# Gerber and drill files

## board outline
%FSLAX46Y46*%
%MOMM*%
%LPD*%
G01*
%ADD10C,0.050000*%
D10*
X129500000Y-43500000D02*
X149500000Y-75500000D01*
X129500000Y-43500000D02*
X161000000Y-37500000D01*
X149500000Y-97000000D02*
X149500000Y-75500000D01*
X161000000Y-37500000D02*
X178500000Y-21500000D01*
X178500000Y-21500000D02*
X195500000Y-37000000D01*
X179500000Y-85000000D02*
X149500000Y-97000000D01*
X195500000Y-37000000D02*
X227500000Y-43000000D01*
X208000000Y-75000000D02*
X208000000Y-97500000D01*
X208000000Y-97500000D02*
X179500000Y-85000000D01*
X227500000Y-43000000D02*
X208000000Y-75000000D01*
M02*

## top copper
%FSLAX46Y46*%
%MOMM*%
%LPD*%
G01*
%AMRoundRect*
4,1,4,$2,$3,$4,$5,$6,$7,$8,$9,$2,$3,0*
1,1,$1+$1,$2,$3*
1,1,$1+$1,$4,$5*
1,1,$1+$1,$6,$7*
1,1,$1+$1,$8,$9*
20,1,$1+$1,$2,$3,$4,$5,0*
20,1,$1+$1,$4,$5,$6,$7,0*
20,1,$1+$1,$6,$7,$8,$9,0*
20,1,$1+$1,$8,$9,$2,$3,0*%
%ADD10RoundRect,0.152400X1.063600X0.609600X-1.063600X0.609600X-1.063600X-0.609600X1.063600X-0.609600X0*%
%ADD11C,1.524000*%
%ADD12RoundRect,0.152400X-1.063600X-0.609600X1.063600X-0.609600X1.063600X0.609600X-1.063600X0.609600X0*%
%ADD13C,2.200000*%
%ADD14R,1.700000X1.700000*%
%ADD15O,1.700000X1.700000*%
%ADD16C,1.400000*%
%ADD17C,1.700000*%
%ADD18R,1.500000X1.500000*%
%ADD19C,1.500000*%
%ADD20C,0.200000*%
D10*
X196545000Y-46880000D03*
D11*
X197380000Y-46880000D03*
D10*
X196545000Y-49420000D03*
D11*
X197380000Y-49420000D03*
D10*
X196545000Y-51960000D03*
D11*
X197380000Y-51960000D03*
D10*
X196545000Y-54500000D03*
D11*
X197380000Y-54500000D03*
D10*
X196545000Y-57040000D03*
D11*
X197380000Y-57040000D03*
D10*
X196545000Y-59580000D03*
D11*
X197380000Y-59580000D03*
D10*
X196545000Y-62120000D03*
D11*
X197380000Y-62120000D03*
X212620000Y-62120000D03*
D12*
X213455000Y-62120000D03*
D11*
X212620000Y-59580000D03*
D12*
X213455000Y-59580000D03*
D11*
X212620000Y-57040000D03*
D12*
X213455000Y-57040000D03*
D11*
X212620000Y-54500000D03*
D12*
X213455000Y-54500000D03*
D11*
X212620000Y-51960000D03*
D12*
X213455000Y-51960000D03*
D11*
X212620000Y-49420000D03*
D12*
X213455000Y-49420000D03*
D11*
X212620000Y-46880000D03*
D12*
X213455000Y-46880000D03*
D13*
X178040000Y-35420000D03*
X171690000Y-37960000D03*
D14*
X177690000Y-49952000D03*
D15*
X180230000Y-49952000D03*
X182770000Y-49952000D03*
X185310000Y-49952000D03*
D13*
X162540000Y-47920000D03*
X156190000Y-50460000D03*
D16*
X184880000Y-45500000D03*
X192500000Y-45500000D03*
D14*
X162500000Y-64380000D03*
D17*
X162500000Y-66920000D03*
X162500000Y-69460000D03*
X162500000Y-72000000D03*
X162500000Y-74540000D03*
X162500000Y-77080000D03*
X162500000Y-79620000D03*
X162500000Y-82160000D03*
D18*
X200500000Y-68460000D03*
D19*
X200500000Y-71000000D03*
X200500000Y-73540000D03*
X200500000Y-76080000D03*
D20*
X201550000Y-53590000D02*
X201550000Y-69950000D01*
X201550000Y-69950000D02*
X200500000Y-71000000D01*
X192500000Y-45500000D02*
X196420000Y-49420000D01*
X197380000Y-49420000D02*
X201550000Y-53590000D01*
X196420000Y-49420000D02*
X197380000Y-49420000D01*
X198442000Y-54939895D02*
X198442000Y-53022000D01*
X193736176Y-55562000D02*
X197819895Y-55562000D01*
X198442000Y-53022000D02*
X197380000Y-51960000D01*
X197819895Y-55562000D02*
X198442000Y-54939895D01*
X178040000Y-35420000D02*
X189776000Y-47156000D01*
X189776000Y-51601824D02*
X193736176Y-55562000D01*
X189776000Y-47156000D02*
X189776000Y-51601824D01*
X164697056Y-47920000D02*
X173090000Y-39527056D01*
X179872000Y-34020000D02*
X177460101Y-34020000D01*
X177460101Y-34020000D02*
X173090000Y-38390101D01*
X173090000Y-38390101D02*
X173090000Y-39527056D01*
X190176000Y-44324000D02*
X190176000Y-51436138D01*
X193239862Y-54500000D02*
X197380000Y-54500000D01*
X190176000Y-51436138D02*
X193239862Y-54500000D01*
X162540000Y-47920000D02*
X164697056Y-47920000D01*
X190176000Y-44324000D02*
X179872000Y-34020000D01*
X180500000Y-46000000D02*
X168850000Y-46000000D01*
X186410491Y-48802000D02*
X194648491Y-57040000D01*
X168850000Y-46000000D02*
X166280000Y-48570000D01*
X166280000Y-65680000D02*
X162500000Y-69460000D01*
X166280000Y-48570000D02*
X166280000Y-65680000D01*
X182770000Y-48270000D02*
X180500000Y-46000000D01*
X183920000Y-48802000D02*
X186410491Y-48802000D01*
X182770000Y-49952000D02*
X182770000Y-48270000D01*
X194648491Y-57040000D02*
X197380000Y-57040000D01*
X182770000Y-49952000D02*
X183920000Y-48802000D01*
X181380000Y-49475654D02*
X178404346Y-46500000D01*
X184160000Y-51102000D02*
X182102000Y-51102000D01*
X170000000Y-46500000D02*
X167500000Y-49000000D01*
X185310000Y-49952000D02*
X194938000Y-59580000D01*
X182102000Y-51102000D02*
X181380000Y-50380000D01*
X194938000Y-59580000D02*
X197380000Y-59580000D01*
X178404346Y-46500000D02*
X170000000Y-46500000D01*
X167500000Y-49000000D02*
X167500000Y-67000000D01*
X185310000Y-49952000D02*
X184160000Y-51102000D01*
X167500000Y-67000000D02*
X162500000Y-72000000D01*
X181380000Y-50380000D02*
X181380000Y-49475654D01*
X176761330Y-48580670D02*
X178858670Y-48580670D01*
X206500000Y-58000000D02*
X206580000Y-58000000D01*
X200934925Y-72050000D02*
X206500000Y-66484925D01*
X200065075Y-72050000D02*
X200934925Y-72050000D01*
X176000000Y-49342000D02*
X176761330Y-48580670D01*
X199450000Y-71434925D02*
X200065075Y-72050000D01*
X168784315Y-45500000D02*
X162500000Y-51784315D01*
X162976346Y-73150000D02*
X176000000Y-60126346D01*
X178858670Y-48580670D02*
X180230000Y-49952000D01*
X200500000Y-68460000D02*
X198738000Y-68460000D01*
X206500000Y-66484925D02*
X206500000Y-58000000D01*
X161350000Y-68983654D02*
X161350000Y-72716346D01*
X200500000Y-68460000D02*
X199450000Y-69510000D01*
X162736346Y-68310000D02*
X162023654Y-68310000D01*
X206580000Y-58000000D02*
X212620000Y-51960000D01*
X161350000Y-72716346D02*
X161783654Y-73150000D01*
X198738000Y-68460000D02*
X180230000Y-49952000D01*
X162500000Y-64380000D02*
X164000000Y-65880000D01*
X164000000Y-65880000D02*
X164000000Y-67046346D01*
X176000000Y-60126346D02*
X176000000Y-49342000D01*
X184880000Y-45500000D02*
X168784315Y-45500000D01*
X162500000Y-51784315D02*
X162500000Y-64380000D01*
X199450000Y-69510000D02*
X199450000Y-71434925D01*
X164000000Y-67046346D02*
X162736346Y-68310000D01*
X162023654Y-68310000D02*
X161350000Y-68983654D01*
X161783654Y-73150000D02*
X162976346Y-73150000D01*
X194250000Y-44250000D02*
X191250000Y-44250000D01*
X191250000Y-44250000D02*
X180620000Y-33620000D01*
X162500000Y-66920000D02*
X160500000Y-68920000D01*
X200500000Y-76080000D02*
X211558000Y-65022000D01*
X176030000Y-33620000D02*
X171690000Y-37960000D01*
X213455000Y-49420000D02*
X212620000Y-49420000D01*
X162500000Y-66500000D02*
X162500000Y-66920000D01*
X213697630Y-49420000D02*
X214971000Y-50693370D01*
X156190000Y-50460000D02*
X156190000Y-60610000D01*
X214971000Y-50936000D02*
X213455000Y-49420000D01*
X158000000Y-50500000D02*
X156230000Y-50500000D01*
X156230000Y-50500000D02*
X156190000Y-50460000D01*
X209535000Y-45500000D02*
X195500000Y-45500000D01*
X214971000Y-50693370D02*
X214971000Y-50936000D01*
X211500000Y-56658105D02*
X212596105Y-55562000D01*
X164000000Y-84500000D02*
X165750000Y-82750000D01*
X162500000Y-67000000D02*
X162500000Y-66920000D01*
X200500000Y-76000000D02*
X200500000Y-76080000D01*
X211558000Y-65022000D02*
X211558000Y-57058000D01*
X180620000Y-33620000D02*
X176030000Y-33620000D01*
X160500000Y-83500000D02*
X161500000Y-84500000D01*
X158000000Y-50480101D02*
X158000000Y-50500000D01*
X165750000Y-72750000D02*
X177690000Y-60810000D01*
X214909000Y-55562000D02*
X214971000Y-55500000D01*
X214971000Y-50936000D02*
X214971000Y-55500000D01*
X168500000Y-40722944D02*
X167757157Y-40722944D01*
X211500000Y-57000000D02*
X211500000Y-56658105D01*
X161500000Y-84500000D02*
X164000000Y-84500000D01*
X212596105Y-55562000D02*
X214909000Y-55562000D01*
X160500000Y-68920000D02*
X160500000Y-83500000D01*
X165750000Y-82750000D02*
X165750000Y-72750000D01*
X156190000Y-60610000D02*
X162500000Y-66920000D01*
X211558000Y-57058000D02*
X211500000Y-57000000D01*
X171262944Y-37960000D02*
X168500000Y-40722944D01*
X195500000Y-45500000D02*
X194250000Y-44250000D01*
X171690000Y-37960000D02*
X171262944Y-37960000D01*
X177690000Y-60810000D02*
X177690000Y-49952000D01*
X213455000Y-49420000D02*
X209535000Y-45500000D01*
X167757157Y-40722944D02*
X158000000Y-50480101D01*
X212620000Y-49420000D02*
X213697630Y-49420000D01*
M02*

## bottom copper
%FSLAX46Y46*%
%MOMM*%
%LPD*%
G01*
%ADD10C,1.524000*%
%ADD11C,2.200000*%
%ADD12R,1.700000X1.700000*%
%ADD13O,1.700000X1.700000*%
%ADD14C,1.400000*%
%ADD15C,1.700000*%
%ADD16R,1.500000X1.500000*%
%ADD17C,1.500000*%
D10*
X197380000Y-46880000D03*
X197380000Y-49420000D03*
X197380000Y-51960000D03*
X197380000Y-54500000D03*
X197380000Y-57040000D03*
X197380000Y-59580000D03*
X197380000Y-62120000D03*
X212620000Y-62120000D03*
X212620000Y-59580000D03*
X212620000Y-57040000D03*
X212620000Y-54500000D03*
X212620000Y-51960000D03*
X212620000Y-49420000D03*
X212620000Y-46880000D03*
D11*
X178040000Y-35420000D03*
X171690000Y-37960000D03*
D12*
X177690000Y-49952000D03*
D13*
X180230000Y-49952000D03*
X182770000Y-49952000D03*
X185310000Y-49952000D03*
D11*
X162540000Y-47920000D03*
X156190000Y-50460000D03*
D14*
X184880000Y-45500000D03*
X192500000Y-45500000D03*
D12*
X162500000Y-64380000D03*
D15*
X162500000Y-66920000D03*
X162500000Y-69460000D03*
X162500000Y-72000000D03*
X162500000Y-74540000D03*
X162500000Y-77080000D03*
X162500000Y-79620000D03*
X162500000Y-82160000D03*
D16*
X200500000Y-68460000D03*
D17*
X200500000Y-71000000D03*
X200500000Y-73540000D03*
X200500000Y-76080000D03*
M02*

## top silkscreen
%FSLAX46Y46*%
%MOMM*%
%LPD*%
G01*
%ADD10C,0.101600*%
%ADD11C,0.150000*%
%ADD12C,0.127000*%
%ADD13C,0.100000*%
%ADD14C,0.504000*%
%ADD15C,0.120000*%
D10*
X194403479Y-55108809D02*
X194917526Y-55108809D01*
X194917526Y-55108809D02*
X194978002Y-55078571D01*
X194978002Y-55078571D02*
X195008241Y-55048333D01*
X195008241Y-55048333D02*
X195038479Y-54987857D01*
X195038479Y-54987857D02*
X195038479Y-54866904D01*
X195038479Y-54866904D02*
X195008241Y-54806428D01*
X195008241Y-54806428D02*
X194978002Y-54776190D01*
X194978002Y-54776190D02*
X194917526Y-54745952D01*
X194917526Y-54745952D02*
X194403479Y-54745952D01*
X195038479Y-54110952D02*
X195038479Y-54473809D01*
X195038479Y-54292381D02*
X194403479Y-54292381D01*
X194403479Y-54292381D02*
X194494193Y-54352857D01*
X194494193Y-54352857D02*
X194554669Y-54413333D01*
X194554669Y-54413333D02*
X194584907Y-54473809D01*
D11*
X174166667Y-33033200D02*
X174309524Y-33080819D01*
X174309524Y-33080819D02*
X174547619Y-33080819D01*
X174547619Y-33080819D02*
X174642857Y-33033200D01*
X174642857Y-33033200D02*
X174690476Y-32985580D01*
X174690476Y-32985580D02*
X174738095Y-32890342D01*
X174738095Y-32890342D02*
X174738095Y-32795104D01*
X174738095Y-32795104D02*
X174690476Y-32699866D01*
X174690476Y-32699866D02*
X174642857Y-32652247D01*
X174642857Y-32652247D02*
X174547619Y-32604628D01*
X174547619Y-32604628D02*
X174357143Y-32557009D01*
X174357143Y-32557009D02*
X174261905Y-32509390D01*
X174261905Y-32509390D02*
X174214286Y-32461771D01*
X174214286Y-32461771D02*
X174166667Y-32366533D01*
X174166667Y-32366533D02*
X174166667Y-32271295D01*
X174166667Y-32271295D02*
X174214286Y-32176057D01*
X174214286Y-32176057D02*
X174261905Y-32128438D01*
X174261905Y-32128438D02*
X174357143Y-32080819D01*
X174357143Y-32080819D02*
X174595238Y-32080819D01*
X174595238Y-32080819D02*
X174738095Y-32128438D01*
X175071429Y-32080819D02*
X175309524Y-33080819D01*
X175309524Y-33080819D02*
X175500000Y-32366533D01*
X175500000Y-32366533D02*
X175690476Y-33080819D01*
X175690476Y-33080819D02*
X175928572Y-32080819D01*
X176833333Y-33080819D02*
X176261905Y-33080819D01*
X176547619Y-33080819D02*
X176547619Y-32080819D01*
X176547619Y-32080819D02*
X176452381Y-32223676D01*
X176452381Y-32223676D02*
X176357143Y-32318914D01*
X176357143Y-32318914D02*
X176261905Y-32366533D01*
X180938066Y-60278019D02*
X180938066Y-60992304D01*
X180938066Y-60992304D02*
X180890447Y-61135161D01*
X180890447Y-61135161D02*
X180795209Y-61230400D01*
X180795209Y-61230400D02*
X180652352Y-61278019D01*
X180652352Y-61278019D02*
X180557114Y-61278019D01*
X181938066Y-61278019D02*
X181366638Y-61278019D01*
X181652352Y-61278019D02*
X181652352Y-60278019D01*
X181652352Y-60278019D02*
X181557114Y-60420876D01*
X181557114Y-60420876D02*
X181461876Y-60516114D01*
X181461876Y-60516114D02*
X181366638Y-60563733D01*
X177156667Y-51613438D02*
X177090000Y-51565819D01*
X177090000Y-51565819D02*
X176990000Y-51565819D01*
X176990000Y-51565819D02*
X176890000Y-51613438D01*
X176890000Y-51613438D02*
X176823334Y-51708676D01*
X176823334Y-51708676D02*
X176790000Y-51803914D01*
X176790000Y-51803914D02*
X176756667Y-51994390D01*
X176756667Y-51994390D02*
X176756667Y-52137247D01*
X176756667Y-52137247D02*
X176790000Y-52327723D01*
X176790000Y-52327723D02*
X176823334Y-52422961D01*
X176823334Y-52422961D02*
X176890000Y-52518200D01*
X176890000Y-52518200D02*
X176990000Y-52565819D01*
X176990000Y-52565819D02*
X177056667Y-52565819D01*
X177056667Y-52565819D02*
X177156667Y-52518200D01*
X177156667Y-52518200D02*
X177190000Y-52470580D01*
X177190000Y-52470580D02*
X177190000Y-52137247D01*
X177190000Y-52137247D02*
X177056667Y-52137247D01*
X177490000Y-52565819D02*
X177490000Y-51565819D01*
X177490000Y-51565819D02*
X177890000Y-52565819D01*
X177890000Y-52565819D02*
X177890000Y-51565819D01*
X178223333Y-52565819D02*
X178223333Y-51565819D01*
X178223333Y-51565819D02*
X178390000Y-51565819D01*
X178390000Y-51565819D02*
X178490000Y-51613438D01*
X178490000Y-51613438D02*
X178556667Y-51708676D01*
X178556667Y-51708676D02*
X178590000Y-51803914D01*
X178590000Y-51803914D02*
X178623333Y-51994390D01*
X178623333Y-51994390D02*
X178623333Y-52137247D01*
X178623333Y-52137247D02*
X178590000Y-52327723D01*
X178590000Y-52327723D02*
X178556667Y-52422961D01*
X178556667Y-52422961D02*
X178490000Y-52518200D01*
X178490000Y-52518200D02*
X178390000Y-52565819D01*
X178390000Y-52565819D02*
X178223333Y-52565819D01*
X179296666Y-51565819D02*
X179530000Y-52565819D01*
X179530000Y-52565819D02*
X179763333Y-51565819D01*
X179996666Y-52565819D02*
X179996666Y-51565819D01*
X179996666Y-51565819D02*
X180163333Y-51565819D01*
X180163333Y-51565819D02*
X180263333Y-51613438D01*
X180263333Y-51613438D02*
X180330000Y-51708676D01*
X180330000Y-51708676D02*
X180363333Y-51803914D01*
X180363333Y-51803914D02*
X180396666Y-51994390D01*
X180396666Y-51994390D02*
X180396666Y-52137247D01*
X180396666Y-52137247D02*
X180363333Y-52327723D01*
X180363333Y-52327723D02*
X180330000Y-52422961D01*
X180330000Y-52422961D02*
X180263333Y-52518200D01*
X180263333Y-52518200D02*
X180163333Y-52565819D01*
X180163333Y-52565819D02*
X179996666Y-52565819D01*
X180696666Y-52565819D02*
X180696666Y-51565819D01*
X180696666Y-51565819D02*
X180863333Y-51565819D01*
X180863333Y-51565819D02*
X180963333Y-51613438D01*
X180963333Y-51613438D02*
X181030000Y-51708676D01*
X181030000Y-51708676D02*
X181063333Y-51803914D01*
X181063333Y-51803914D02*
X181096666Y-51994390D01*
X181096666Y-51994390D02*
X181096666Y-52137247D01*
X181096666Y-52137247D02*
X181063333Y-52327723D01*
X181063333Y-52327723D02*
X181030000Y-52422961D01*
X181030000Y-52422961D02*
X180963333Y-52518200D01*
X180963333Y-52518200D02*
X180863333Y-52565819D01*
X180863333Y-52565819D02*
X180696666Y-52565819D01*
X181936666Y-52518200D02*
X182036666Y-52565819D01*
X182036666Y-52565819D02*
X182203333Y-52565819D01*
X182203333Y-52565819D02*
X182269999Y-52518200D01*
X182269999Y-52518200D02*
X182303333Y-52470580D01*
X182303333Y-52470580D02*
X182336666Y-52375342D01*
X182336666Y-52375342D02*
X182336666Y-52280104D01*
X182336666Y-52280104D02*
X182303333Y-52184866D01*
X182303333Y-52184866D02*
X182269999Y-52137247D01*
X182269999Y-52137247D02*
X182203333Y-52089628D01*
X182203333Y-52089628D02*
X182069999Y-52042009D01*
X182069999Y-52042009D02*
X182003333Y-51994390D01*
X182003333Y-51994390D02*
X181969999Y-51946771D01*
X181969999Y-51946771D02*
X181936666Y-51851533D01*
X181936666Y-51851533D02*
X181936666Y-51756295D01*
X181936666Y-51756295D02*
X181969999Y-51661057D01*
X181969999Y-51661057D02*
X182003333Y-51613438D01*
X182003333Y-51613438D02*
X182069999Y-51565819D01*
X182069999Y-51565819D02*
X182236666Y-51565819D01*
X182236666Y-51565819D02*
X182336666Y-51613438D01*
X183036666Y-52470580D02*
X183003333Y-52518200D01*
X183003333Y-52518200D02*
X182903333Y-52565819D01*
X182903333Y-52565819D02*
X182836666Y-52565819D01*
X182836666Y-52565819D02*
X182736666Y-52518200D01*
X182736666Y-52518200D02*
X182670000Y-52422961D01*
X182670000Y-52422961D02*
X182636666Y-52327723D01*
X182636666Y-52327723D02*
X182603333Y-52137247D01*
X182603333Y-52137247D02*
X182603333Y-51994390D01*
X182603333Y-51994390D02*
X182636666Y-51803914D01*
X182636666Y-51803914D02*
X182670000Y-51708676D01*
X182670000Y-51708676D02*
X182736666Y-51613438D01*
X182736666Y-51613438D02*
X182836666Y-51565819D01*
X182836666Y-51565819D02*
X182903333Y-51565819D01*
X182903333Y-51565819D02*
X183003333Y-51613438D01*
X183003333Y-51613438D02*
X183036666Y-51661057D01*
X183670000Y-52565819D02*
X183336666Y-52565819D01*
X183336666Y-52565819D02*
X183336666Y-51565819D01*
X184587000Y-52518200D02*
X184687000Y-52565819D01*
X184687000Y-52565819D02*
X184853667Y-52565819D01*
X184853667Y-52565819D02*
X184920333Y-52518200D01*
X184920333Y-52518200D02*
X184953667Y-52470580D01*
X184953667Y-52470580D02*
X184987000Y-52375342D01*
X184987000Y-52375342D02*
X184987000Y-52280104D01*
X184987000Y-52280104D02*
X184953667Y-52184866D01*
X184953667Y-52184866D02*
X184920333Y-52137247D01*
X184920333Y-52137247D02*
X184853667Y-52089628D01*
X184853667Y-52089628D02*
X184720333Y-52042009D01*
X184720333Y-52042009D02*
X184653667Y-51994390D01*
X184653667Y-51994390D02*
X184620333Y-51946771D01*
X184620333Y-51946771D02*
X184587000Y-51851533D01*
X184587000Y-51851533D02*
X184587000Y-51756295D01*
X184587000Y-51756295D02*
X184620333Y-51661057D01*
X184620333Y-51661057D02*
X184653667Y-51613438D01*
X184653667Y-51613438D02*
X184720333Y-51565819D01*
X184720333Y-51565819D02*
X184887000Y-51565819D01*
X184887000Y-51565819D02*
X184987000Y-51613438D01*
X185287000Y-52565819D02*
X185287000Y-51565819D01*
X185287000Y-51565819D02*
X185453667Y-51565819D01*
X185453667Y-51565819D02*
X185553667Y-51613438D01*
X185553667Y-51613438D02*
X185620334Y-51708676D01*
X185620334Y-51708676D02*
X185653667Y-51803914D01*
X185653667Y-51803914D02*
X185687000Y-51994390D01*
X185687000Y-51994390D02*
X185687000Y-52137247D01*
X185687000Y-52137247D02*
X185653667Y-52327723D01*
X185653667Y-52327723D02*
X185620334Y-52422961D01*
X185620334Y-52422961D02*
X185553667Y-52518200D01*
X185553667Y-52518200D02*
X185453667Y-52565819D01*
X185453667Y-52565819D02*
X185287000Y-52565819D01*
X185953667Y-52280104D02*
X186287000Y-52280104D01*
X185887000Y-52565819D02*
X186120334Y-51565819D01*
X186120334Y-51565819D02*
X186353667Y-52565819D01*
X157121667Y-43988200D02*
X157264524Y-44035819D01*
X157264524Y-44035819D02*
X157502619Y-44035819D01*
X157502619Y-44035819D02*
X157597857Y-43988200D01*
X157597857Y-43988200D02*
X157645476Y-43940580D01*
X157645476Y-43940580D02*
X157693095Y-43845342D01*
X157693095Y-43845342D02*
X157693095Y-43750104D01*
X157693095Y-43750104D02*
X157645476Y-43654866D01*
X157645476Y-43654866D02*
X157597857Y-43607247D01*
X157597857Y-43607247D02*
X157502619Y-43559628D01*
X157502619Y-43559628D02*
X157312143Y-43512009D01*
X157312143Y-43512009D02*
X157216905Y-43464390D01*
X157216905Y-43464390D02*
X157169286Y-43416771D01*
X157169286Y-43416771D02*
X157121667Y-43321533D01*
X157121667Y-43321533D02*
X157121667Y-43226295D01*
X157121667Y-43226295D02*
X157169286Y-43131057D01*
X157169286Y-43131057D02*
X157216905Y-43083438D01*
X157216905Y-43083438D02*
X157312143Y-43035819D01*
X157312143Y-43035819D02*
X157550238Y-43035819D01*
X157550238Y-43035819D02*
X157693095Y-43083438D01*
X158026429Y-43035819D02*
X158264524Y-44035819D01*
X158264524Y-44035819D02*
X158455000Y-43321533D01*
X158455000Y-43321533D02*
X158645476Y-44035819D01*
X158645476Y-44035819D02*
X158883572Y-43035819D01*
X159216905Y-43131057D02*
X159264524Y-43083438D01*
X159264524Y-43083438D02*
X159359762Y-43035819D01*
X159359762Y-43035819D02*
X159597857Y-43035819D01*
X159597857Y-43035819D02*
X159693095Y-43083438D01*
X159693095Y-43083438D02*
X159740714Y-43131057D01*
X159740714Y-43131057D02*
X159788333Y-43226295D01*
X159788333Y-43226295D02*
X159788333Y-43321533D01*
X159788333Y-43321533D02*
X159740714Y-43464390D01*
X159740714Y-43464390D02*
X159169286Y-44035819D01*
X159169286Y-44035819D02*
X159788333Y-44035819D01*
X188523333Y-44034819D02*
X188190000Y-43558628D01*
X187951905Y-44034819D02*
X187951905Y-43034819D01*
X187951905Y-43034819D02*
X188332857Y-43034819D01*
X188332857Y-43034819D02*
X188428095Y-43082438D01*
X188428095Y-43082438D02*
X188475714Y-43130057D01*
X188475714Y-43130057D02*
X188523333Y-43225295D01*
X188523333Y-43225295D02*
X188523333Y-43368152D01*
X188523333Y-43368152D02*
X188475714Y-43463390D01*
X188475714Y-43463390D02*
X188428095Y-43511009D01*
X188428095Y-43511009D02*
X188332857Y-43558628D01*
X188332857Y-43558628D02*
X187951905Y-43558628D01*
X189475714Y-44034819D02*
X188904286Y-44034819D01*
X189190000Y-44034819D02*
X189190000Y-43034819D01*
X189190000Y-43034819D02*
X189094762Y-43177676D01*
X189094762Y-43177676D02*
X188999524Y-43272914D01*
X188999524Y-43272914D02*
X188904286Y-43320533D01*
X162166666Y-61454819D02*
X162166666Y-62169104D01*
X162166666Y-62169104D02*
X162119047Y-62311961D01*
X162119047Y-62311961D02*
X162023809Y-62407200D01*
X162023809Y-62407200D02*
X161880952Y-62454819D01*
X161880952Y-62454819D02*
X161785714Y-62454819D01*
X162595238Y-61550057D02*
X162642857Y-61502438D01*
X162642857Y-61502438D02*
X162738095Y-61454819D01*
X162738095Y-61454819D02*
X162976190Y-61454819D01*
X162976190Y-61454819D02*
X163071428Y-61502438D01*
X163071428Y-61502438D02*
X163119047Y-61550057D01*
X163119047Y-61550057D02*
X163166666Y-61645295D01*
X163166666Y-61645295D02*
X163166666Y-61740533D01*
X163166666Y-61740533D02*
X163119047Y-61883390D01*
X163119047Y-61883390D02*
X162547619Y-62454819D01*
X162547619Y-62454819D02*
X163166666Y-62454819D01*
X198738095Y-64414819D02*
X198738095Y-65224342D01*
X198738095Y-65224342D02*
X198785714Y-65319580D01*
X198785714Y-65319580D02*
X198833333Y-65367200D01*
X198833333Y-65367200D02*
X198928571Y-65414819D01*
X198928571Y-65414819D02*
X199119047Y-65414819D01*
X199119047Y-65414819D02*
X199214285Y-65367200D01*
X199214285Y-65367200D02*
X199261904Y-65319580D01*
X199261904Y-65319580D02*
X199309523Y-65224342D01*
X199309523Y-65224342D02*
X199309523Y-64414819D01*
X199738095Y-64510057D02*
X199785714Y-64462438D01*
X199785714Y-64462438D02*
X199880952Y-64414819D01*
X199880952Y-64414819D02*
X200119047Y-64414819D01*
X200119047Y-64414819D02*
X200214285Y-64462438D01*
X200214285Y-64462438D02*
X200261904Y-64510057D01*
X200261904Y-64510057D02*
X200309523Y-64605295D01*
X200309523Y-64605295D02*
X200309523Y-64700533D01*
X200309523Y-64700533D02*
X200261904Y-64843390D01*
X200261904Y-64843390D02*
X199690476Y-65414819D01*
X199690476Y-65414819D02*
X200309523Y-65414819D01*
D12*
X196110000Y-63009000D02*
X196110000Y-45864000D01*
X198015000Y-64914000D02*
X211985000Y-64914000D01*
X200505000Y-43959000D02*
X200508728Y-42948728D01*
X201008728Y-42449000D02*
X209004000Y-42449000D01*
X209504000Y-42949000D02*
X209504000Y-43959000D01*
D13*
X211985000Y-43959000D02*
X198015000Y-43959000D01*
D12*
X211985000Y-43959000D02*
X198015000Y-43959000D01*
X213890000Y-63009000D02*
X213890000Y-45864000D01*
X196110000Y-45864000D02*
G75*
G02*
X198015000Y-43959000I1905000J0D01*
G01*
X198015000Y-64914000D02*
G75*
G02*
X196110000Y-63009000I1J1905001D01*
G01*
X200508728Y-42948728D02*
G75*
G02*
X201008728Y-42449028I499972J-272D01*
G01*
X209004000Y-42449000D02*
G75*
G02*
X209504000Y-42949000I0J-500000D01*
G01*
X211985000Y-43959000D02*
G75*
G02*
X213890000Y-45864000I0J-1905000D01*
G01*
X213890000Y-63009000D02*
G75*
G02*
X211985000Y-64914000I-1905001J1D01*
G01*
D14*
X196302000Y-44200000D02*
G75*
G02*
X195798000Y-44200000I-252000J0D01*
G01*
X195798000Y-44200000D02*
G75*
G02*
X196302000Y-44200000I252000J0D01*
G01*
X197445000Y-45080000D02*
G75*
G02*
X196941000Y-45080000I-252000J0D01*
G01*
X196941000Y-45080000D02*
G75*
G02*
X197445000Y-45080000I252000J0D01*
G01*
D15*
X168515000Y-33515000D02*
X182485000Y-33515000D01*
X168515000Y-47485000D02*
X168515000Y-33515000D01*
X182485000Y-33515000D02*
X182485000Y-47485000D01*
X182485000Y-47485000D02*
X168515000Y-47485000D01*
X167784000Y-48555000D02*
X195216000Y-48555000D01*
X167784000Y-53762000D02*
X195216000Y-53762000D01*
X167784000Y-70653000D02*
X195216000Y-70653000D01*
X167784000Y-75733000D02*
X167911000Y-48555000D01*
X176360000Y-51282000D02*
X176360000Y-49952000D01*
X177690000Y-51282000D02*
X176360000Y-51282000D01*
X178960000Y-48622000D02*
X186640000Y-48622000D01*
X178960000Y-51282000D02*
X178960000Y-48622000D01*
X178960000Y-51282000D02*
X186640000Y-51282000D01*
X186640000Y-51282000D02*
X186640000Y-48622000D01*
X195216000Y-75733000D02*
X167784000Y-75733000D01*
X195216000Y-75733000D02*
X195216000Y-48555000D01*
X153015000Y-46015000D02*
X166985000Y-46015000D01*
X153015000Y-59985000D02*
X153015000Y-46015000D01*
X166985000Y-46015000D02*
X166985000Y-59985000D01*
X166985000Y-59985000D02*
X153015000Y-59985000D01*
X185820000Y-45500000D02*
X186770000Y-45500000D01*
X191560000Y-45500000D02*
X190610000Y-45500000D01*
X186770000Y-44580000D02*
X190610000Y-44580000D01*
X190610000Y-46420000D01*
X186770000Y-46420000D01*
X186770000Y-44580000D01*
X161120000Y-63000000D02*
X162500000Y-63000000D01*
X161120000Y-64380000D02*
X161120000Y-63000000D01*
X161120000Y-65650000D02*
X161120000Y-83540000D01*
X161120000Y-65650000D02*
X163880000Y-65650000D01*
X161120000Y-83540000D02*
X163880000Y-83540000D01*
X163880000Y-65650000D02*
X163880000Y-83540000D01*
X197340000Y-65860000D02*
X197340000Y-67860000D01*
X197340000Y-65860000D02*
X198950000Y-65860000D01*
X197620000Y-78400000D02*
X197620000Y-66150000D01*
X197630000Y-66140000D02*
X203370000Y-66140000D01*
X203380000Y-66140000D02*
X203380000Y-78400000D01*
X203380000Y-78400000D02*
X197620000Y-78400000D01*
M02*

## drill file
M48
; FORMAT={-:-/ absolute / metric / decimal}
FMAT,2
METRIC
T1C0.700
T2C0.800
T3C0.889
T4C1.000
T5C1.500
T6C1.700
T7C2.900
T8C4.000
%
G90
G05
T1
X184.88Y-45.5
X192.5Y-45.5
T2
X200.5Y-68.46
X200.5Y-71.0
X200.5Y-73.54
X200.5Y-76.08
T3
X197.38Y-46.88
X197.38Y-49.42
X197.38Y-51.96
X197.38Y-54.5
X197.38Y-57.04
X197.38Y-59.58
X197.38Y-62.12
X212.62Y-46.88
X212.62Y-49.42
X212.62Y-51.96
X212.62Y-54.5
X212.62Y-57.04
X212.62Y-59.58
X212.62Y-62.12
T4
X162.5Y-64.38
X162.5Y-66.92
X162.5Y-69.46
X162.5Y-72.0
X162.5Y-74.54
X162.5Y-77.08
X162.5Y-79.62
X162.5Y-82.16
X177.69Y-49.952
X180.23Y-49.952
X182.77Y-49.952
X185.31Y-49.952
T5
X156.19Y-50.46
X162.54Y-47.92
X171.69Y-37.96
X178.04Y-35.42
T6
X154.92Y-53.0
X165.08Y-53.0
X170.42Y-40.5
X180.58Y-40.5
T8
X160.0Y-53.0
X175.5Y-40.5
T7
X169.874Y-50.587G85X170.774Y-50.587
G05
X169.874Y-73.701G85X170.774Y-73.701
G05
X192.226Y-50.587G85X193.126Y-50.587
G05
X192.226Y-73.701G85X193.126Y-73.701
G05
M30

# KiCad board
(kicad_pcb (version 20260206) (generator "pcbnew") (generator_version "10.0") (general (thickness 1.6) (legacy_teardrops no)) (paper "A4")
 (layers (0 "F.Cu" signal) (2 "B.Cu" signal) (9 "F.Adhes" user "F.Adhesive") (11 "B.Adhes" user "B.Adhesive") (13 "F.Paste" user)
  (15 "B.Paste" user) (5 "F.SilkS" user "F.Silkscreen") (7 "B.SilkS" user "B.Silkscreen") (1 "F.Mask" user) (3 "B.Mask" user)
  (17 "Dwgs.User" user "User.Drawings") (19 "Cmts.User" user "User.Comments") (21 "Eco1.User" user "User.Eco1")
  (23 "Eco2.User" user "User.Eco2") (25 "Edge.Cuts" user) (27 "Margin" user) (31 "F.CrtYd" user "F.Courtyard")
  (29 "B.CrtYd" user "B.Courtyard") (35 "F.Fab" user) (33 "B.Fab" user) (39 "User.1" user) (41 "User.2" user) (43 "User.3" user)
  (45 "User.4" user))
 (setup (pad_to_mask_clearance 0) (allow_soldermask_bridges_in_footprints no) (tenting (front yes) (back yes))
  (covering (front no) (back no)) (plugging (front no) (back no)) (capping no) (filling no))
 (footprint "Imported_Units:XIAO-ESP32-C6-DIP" (layer "F.Cu") (at 205 54.5 90)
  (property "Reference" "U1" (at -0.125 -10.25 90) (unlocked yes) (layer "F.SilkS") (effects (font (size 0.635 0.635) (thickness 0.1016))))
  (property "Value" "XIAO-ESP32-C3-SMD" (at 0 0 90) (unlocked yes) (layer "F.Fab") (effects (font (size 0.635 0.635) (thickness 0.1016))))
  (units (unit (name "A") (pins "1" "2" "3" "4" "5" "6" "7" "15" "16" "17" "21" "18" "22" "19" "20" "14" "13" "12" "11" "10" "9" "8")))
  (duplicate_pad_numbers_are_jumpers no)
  (fp_line (start -8.509 -8.89) (end 8.636 -8.89) (stroke (width 0.127) (type solid)) (layer "F.SilkS"))
  (fp_line (start -10.414 -6.985) (end -10.414 6.985) (stroke (width 0.127) (type solid)) (layer "F.SilkS"))
  (fp_line (start 10.541 -4.495) (end 11.551272 -4.491272) (stroke (width 0.127) (type solid)) (layer "F.SilkS"))
  (fp_line (start 12.051 -3.991272) (end 12.051 4.004) (stroke (width 0.127) (type solid)) (layer "F.SilkS"))
  (fp_line (start 11.551 4.504) (end 10.541 4.504) (stroke (width 0.127) (type solid)) (layer "F.SilkS"))
  (fp_line (start 10.541 6.985) (end 10.541 -6.985) (stroke (width 0.1) (type solid)) (layer "F.SilkS"))
  (fp_line (start 10.541 6.985) (end 10.541 -6.985) (stroke (width 0.127) (type solid)) (layer "F.SilkS"))
  (fp_line (start -8.509 8.89) (end 8.636 8.89) (stroke (width 0.127) (type solid)) (layer "F.SilkS"))
  (fp_arc (start 8.636 -8.89) (mid 9.983038 -8.332038) (end 10.541 -6.985) (stroke (width 0.127) (type solid)) (layer "F.SilkS"))
  (fp_arc (start -10.414 -6.985) (mid -9.856038 -8.332038) (end -8.509 -8.89) (stroke (width 0.127) (type solid)) (layer "F.SilkS"))
  (fp_arc (start 11.551272 -4.491272) (mid 11.904644 -4.344724) (end 12.051 -3.991272) (stroke (width 0.127) (type default))
   (layer "F.SilkS"))
  (fp_arc (start 12.051 4.004) (mid 11.904553 4.357553) (end 11.551 4.504) (stroke (width 0.127) (type default)) (layer "F.SilkS"))
  (fp_arc (start 10.541 6.985) (mid 9.983038 8.332038) (end 8.636 8.89) (stroke (width 0.127) (type solid)) (layer "F.SilkS"))
  (fp_arc (start -8.509 8.89) (mid -9.856038 8.332038) (end -10.414 6.985) (stroke (width 0.127) (type solid)) (layer "F.SilkS"))
  (fp_circle (center 10.3 -8.95) (end 10.554 -8.95) (stroke (width 0.5) (type solid)) (fill yes) (layer "F.SilkS"))
  (fp_circle (center 9.42 -7.807) (end 9.674 -7.807) (stroke (width 0.5) (type solid)) (fill yes) (layer "F.SilkS"))
  (pad "1" smd roundrect (at 7.62 -8.455 180) (size 2.432 1.524) (layers "F.Cu" "F.Mask") (roundrect_rratio 0.1)
   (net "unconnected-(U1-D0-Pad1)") (thermal_bridge_angle 45))
  (pad "1" thru_hole circle (at 7.62 -7.62 180) (size 1.524 1.524) (drill 0.889) (layers "*.Cu" "*.Mask") (remove_unused_layers no)
   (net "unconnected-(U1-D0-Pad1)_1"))
  (pad "2" smd roundrect (at 5.08 -8.455 180) (size 2.432 1.524) (layers "F.Cu" "F.Mask") (roundrect_rratio 0.1) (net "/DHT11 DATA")
   (thermal_bridge_angle 45))
  (pad "2" thru_hole circle (at 5.08 -7.62 180) (size 1.524 1.524) (drill 0.889) (layers "*.Cu" "*.Mask") (remove_unused_layers no)
   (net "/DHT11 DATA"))
  (pad "3" smd roundrect (at 2.54 -8.455 180) (size 2.432 1.524) (layers "F.Cu" "F.Mask") (roundrect_rratio 0.1) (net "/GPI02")
   (thermal_bridge_angle 45))
  (pad "3" thru_hole circle (at 2.54 -7.62 180) (size 1.524 1.524) (drill 0.889) (layers "*.Cu" "*.Mask") (remove_unused_layers no)
   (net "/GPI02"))
  (pad "4" smd roundrect (at 0 -8.455 180) (size 2.432 1.524) (layers "F.Cu" "F.Mask") (roundrect_rratio 0.1) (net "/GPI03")
   (thermal_bridge_angle 45))
  (pad "4" thru_hole circle (at 0 -7.62 180) (size 1.524 1.524) (drill 0.889) (layers "*.Cu" "*.Mask") (remove_unused_layers no)
   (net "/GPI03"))
  (pad "5" smd roundrect (at -2.54 -8.455 180) (size 2.432 1.524) (layers "F.Cu" "F.Mask") (roundrect_rratio 0.1) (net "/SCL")
   (thermal_bridge_angle 45))
  (pad "5" thru_hole circle (at -2.54 -7.62 180) (size 1.524 1.524) (drill 0.889) (layers "*.Cu" "*.Mask") (remove_unused_layers no)
   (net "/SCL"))
  (pad "6" smd roundrect (at -5.08 -8.455 180) (size 2.432 1.524) (layers "F.Cu" "F.Mask") (roundrect_rratio 0.1) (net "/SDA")
   (thermal_bridge_angle 45))
  (pad "6" thru_hole circle (at -5.08 -7.62 180) (size 1.524 1.524) (drill 0.889) (layers "*.Cu" "*.Mask") (remove_unused_layers no)
   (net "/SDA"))
  (pad "7" smd roundrect (at -7.62 -8.455 180) (size 2.432 1.524) (layers "F.Cu" "F.Mask") (roundrect_rratio 0.1)
   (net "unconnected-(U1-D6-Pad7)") (thermal_bridge_angle 45))
  (pad "7" thru_hole circle (at -7.62 -7.62 180) (size 1.524 1.524) (drill 0.889) (layers "*.Cu" "*.Mask") (remove_unused_layers no)
   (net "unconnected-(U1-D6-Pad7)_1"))
  (pad "8" thru_hole circle (at -7.62 7.62) (size 1.524 1.524) (drill 0.889) (layers "*.Cu" "*.Mask") (remove_unused_layers no)
   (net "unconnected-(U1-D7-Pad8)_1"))
  (pad "8" smd roundrect (at -7.62 8.455) (size 2.432 1.524) (layers "F.Cu" "F.Mask") (roundrect_rratio 0.1)
   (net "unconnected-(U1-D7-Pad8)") (thermal_bridge_angle 45))
  (pad "9" thru_hole circle (at -5.08 7.62) (size 1.524 1.524) (drill 0.889) (layers "*.Cu" "*.Mask") (remove_unused_layers no)
   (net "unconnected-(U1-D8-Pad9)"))
  (pad "9" smd roundrect (at -5.08 8.455) (size 2.432 1.524) (layers "F.Cu" "F.Mask") (roundrect_rratio 0.1)
   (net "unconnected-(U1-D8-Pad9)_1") (thermal_bridge_angle 45))
  (pad "10" thru_hole circle (at -2.54 7.62) (size 1.524 1.524) (drill 0.889) (layers "*.Cu" "*.Mask") (remove_unused_layers no)
   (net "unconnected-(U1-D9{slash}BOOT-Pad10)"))
  (pad "10" smd roundrect (at -2.54 8.455) (size 2.432 1.524) (layers "F.Cu" "F.Mask") (roundrect_rratio 0.1)
   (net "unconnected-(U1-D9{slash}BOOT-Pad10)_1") (thermal_bridge_angle 45))
  (pad "11" thru_hole circle (at 0 7.62) (size 1.524 1.524) (drill 0.889) (layers "*.Cu" "*.Mask") (remove_unused_layers no)
   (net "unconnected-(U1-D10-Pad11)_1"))
  (pad "11" smd roundrect (at 0 8.455) (size 2.432 1.524) (layers "F.Cu" "F.Mask") (roundrect_rratio 0.1) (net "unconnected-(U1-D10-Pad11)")
   (thermal_bridge_angle 45))
  (pad "12" thru_hole circle (at 2.54 7.62) (size 1.524 1.524) (drill 0.889) (layers "*.Cu" "*.Mask") (remove_unused_layers no)
   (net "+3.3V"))
  (pad "12" smd roundrect (at 2.54 8.455) (size 2.432 1.524) (layers "F.Cu" "F.Mask") (roundrect_rratio 0.1) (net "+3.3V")
   (thermal_bridge_angle 45))
  (pad "13" thru_hole circle (at 5.08 7.62) (size 1.524 1.524) (drill 0.889) (layers "*.Cu" "*.Mask") (remove_unused_layers no) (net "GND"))
  (pad "13" smd roundrect (at 5.08 8.455) (size 2.432 1.524) (layers "F.Cu" "F.Mask") (roundrect_rratio 0.1) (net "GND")
   (thermal_bridge_angle 45))
  (pad "14" thru_hole circle (at 7.62 7.62) (size 1.524 1.524) (drill 0.889) (layers "*.Cu" "*.Mask") (remove_unused_layers no) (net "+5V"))
  (pad "14" smd roundrect (at 7.62 8.455) (size 2.432 1.524) (layers "F.Cu" "F.Mask") (roundrect_rratio 0.1) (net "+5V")
   (thermal_bridge_angle 45)))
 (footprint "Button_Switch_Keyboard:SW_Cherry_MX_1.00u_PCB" (layer "F.Cu") (at 178.04 35.42)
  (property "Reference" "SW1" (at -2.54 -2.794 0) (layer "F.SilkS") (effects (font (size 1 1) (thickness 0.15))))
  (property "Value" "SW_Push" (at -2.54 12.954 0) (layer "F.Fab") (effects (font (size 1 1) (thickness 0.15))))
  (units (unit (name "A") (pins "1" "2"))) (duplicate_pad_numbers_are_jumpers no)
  (fp_line (start -9.525 -1.905) (end 4.445 -1.905) (stroke (width 0.12) (type solid)) (layer "F.SilkS"))
  (fp_line (start -9.525 12.065) (end -9.525 -1.905) (stroke (width 0.12) (type solid)) (layer "F.SilkS"))
  (fp_line (start 4.445 -1.905) (end 4.445 12.065) (stroke (width 0.12) (type solid)) (layer "F.SilkS"))
  (fp_line (start 4.445 12.065) (end -9.525 12.065) (stroke (width 0.12) (type solid)) (layer "F.SilkS"))
  (pad "" np_thru_hole circle (at -7.62 5.08) (size 1.7 1.7) (drill 1.7) (layers "*.Cu" "*.Mask"))
  (pad "" np_thru_hole circle (at -2.54 5.08) (size 4 4) (drill 4) (layers "*.Cu" "*.Mask"))
  (pad "" np_thru_hole circle (at 2.54 5.08) (size 1.7 1.7) (drill 1.7) (layers "*.Cu" "*.Mask"))
  (pad "1" thru_hole circle (at 0 0) (size 2.2 2.2) (drill 1.5) (layers "*.Cu" "*.Mask") (remove_unused_layers no) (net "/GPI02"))
  (pad "2" thru_hole circle (at -6.35 2.54) (size 2.2 2.2) (drill 1.5) (layers "*.Cu" "*.Mask") (remove_unused_layers no) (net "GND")))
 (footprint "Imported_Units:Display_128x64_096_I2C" (layer "F.Cu") (at 181.5 49.952)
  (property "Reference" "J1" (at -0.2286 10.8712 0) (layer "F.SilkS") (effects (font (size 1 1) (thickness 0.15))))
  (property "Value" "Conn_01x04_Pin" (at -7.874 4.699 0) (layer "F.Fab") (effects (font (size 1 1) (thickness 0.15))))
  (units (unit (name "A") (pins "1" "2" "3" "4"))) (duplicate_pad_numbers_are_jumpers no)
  (fp_line (start -13.716 -1.397) (end 13.716 -1.397) (stroke (width 0.12) (type solid)) (layer "F.SilkS"))
  (fp_line (start -13.716 3.81) (end 13.716 3.81) (stroke (width 0.12) (type solid)) (layer "F.SilkS"))
  (fp_line (start -13.716 20.701) (end 13.716 20.701) (stroke (width 0.12) (type solid)) (layer "F.SilkS"))
  (fp_line (start -13.716 25.781) (end -13.589 -1.397) (stroke (width 0.12) (type solid)) (layer "F.SilkS"))
  (fp_line (start -5.14 1.33) (end -5.14 0) (stroke (width 0.12) (type solid)) (layer "F.SilkS"))
  (fp_line (start -3.81 1.33) (end -5.14 1.33) (stroke (width 0.12) (type solid)) (layer "F.SilkS"))
  (fp_line (start -2.54 -1.33) (end 5.14 -1.33) (stroke (width 0.12) (type solid)) (layer "F.SilkS"))
  (fp_line (start -2.54 1.33) (end -2.54 -1.33) (stroke (width 0.12) (type solid)) (layer "F.SilkS"))
  (fp_line (start -2.54 1.33) (end 5.14 1.33) (stroke (width 0.12) (type solid)) (layer "F.SilkS"))
  (fp_line (start 5.14 1.33) (end 5.14 -1.33) (stroke (width 0.12) (type solid)) (layer "F.SilkS"))
  (fp_line (start 13.716 25.781) (end -13.716 25.781) (stroke (width 0.12) (type solid)) (layer "F.SilkS"))
  (fp_line (start 13.716 25.781) (end 13.716 -1.397) (stroke (width 0.12) (type solid)) (layer "F.SilkS"))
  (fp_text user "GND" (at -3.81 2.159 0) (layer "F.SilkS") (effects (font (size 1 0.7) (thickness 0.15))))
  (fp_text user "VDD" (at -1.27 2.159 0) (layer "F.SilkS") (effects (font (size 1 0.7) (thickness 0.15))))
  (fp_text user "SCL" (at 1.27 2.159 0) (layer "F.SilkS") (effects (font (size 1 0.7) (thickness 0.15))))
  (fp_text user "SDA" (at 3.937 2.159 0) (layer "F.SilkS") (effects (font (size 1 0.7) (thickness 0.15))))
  (pad "" np_thru_hole oval (at -11.176 0.635) (size 3.8 2.9) (drill oval 3.8 2.9) (layers "*.Cu" "*.Mask"))
  (pad "" np_thru_hole oval (at -11.176 23.749) (size 3.8 2.9) (drill oval 3.8 2.9) (layers "*.Cu" "*.Mask"))
  (pad "" np_thru_hole oval (at 11.176 0.635) (size 3.8 2.9) (drill oval 3.8 2.9) (layers "*.Cu" "*.Mask"))
  (pad "" np_thru_hole oval (at 11.176 23.749) (size 3.8 2.9) (drill oval 3.8 2.9) (layers "*.Cu" "*.Mask"))
  (pad "1" thru_hole rect (at -3.81 0 90) (size 1.7 1.7) (drill 1) (layers "*.Cu" "*.Mask") (remove_unused_layers no) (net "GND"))
  (pad "2" thru_hole oval (at -1.27 0 90) (size 1.7 1.7) (drill 1) (layers "*.Cu" "*.Mask") (remove_unused_layers no) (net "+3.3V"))
  (pad "3" thru_hole oval (at 1.27 0 90) (size 1.7 1.7) (drill 1) (layers "*.Cu" "*.Mask") (remove_unused_layers no) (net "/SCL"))
  (pad "4" thru_hole oval (at 3.81 0 90) (size 1.7 1.7) (drill 1) (layers "*.Cu" "*.Mask") (remove_unused_layers no) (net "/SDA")))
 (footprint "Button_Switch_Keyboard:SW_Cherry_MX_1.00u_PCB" (layer "F.Cu") (at 162.54 47.92)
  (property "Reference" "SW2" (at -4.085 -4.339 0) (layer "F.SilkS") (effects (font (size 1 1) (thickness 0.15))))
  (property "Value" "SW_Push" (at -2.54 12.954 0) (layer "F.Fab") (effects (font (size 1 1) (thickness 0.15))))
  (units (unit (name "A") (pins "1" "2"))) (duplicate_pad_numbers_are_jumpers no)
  (fp_line (start -9.525 -1.905) (end 4.445 -1.905) (stroke (width 0.12) (type solid)) (layer "F.SilkS"))
  (fp_line (start -9.525 12.065) (end -9.525 -1.905) (stroke (width 0.12) (type solid)) (layer "F.SilkS"))
  (fp_line (start 4.445 -1.905) (end 4.445 12.065) (stroke (width 0.12) (type solid)) (layer "F.SilkS"))
  (fp_line (start 4.445 12.065) (end -9.525 12.065) (stroke (width 0.12) (type solid)) (layer "F.SilkS"))
  (pad "" np_thru_hole circle (at -7.62 5.08) (size 1.7 1.7) (drill 1.7) (layers "*.Cu" "*.Mask"))
  (pad "" np_thru_hole circle (at -2.54 5.08) (size 4 4) (drill 4) (layers "*.Cu" "*.Mask"))
  (pad "" np_thru_hole circle (at 2.54 5.08) (size 1.7 1.7) (drill 1.7) (layers "*.Cu" "*.Mask"))
  (pad "1" thru_hole circle (at 0 0) (size 2.2 2.2) (drill 1.5) (layers "*.Cu" "*.Mask") (remove_unused_layers no) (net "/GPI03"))
  (pad "2" thru_hole circle (at -6.35 2.54) (size 2.2 2.2) (drill 1.5) (layers "*.Cu" "*.Mask") (remove_unused_layers no) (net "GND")))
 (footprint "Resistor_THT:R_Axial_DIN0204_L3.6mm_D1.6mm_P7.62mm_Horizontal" (layer "F.Cu") (at 184.88 45.5)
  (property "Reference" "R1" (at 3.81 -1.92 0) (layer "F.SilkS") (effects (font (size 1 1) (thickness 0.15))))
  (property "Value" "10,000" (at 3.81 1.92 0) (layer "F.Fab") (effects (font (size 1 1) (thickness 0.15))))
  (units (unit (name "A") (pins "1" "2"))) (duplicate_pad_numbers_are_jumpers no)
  (fp_line (start 0.94 0) (end 1.89 0) (stroke (width 0.12) (type solid)) (layer "F.SilkS"))
  (fp_line (start 6.68 0) (end 5.73 0) (stroke (width 0.12) (type solid)) (layer "F.SilkS"))
  (fp_rect (start 1.89 -0.92) (end 5.73 0.92) (stroke (width 0.12) (type solid)) (fill no) (layer "F.SilkS"))
  (pad "1" thru_hole circle (at 0 0) (size 1.4 1.4) (drill 0.7) (layers "*.Cu" "*.Mask") (remove_unused_layers no) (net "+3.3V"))
  (pad "2" thru_hole circle (at 7.62 0) (size 1.4 1.4) (drill 0.7) (layers "*.Cu" "*.Mask") (remove_unused_layers no) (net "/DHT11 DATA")))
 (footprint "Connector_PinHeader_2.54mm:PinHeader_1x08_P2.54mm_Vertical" (layer "F.Cu") (at 162.5 64.38)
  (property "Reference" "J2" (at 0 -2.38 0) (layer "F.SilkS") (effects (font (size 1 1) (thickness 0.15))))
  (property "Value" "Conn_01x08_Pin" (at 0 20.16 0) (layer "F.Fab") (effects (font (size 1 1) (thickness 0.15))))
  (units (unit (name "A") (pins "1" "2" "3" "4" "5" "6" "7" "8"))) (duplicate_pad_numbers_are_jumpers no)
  (fp_line (start -1.38 -1.38) (end 0 -1.38) (stroke (width 0.12) (type solid)) (layer "F.SilkS"))
  (fp_line (start -1.38 0) (end -1.38 -1.38) (stroke (width 0.12) (type solid)) (layer "F.SilkS"))
  (fp_line (start -1.38 1.27) (end -1.38 19.16) (stroke (width 0.12) (type solid)) (layer "F.SilkS"))
  (fp_line (start -1.38 1.27) (end 1.38 1.27) (stroke (width 0.12) (type solid)) (layer "F.SilkS"))
  (fp_line (start -1.38 19.16) (end 1.38 19.16) (stroke (width 0.12) (type solid)) (layer "F.SilkS"))
  (fp_line (start 1.38 1.27) (end 1.38 19.16) (stroke (width 0.12) (type solid)) (layer "F.SilkS"))
  (pad "1" thru_hole rect (at 0 0) (size 1.7 1.7) (drill 1) (layers "*.Cu" "*.Mask") (remove_unused_layers no) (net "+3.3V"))
  (pad "2" thru_hole circle (at 0 2.54) (size 1.7 1.7) (drill 1) (layers "*.Cu" "*.Mask") (remove_unused_layers no) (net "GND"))
  (pad "3" thru_hole circle (at 0 5.08) (size 1.7 1.7) (drill 1) (layers "*.Cu" "*.Mask") (remove_unused_layers no) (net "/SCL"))
  (pad "4" thru_hole circle (at 0 7.62) (size 1.7 1.7) (drill 1) (layers "*.Cu" "*.Mask") (remove_unused_layers no) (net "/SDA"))
  (pad "5" thru_hole circle (at 0 10.16) (size 1.7 1.7) (drill 1) (layers "*.Cu" "*.Mask") (remove_unused_layers no)
   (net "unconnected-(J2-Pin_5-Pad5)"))
  (pad "6" thru_hole circle (at 0 12.7) (size 1.7 1.7) (drill 1) (layers "*.Cu" "*.Mask") (remove_unused_layers no)
   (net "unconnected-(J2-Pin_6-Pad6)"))
  (pad "7" thru_hole circle (at 0 15.24) (size 1.7 1.7) (drill 1) (layers "*.Cu" "*.Mask") (remove_unused_layers no)
   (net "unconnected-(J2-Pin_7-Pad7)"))
  (pad "8" thru_hole circle (at 0 17.78) (size 1.7 1.7) (drill 1) (layers "*.Cu" "*.Mask") (remove_unused_layers no)
   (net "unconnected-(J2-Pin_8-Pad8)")))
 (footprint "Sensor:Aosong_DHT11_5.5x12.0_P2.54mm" (layer "F.Cu") (at 200.5 68.46)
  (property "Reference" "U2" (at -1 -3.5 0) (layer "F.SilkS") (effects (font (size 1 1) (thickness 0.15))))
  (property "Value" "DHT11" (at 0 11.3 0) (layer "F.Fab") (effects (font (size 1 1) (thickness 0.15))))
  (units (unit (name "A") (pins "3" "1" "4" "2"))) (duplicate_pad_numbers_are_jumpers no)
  (fp_line (start -3.16 -2.6) (end -3.16 -0.6) (stroke (width 0.12) (type solid)) (layer "F.SilkS"))
  (fp_line (start -3.16 -2.6) (end -1.55 -2.6) (stroke (width 0.12) (type solid)) (layer "F.SilkS"))
  (fp_line (start -2.88 9.94) (end -2.88 -2.31) (stroke (width 0.12) (type solid)) (layer "F.SilkS"))
  (fp_line (start -2.87 -2.32) (end 2.87 -2.32) (stroke (width 0.12) (type solid)) (layer "F.SilkS"))
  (fp_line (start 2.88 -2.32) (end 2.88 9.94) (stroke (width 0.12) (type solid)) (layer "F.SilkS"))
  (fp_line (start 2.88 9.94) (end -2.88 9.94) (stroke (width 0.12) (type solid)) (layer "F.SilkS"))
  (pad "1" thru_hole rect (at 0 0) (size 1.5 1.5) (drill 0.8) (layers "*.Cu" "*.Mask") (remove_unused_layers no) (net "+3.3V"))
  (pad "2" thru_hole circle (at 0 2.54) (size 1.5 1.5) (drill 0.8) (layers "*.Cu" "*.Mask") (remove_unused_layers no) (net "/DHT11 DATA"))
  (pad "3" thru_hole circle (at 0 5.08) (size 1.5 1.5) (drill 0.8) (layers "*.Cu" "*.Mask") (remove_unused_layers no)
   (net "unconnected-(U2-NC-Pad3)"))
  (pad "4" thru_hole circle (at 0 7.62) (size 1.5 1.5) (drill 0.8) (layers "*.Cu" "*.Mask") (remove_unused_layers no) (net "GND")))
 (gr_line (start 129.5 43.5) (end 149.5 75.5) (stroke (width 0.05) (type default)) (layer "Edge.Cuts"))
 (gr_line (start 129.5 43.5) (end 161 37.5) (stroke (width 0.05) (type default)) (layer "Edge.Cuts"))
 (gr_line (start 149.5 97) (end 149.5 75.5) (stroke (width 0.05) (type default)) (layer "Edge.Cuts"))
 (gr_line (start 161 37.5) (end 178.5 21.5) (stroke (width 0.05) (type default)) (layer "Edge.Cuts"))
 (gr_line (start 178.5 21.5) (end 195.5 37) (stroke (width 0.05) (type default)) (layer "Edge.Cuts"))
 (gr_line (start 179.5 85) (end 149.5 97) (stroke (width 0.05) (type default)) (layer "Edge.Cuts"))
 (gr_line (start 195.5 37) (end 227.5 43) (stroke (width 0.05) (type default)) (layer "Edge.Cuts"))
 (gr_line (start 208 75) (end 208 97.5) (stroke (width 0.05) (type default)) (layer "Edge.Cuts"))
 (gr_line (start 208 97.5) (end 179.5 85) (stroke (width 0.05) (type default)) (layer "Edge.Cuts"))
 (gr_line (start 227.5 43) (end 208 75) (stroke (width 0.05) (type default)) (layer "Edge.Cuts"))
 (segment (start 201.55 53.59) (end 201.55 69.95) (width 0.2) (layer "F.Cu") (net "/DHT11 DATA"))
 (segment (start 201.55 69.95) (end 200.5 71) (width 0.2) (layer "F.Cu") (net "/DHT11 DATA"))
 (segment (start 192.5 45.5) (end 196.42 49.42) (width 0.2) (layer "F.Cu") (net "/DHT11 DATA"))
 (segment (start 197.38 49.42) (end 201.55 53.59) (width 0.2) (layer "F.Cu") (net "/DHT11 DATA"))
 (segment (start 196.42 49.42) (end 197.38 49.42) (width 0.2) (layer "F.Cu") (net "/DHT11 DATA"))
 (segment (start 198.442 54.939895) (end 198.442 53.022) (width 0.2) (layer "F.Cu") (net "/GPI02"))
 (segment (start 193.736176 55.562) (end 197.819895 55.562) (width 0.2) (layer "F.Cu") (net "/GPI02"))
 (segment (start 198.442 53.022) (end 197.38 51.96) (width 0.2) (layer "F.Cu") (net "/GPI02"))
 (segment (start 197.819895 55.562) (end 198.442 54.939895) (width 0.2) (layer "F.Cu") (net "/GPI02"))
 (segment (start 178.04 35.42) (end 189.776 47.156) (width 0.2) (layer "F.Cu") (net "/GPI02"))
 (segment (start 189.776 51.601824) (end 193.736176 55.562) (width 0.2) (layer "F.Cu") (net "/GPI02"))
 (segment (start 189.776 47.156) (end 189.776 51.601824) (width 0.2) (layer "F.Cu") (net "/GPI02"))
 (segment (start 164.697056 47.92) (end 173.09 39.527056) (width 0.2) (layer "F.Cu") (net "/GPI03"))
 (segment (start 179.872 34.02) (end 177.460101 34.02) (width 0.2) (layer "F.Cu") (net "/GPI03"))
 (segment (start 177.460101 34.02) (end 173.09 38.390101) (width 0.2) (layer "F.Cu") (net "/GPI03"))
 (segment (start 173.09 38.390101) (end 173.09 39.527056) (width 0.2) (layer "F.Cu") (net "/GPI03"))
 (segment (start 190.176 44.324) (end 190.176 51.436138) (width 0.2) (layer "F.Cu") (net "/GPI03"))
 (segment (start 193.239862 54.5) (end 197.38 54.5) (width 0.2) (layer "F.Cu") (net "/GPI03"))
 (segment (start 190.176 51.436138) (end 193.239862 54.5) (width 0.2) (layer "F.Cu") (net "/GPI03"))
 (segment (start 162.54 47.92) (end 164.697056 47.92) (width 0.2) (layer "F.Cu") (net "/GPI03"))
 (segment (start 190.176 44.324) (end 179.872 34.02) (width 0.2) (layer "F.Cu") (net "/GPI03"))
 (segment (start 180.5 46) (end 168.85 46) (width 0.2) (layer "F.Cu") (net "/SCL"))
 (segment (start 186.410491 48.802) (end 194.648491 57.04) (width 0.2) (layer "F.Cu") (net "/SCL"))
 (segment (start 168.85 46) (end 166.28 48.57) (width 0.2) (layer "F.Cu") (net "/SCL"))
 (segment (start 166.28 65.68) (end 162.5 69.46) (width 0.2) (layer "F.Cu") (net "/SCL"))
 (segment (start 166.28 48.57) (end 166.28 65.68) (width 0.2) (layer "F.Cu") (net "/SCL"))
 (segment (start 182.77 48.27) (end 180.5 46) (width 0.2) (layer "F.Cu") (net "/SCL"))
 (segment (start 183.92 48.802) (end 186.410491 48.802) (width 0.2) (layer "F.Cu") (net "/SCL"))
 (segment (start 182.77 49.952) (end 182.77 48.27) (width 0.2) (layer "F.Cu") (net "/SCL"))
 (segment (start 194.648491 57.04) (end 197.38 57.04) (width 0.2) (layer "F.Cu") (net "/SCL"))
 (segment (start 182.77 49.952) (end 183.92 48.802) (width 0.2) (layer "F.Cu") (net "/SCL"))
 (segment (start 181.38 49.475654) (end 178.404346 46.5) (width 0.2) (layer "F.Cu") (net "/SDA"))
 (segment (start 184.16 51.102) (end 182.102 51.102) (width 0.2) (layer "F.Cu") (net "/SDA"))
 (segment (start 170 46.5) (end 167.5 49) (width 0.2) (layer "F.Cu") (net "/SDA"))
 (segment (start 185.31 49.952) (end 194.938 59.58) (width 0.2) (layer "F.Cu") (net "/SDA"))
 (segment (start 182.102 51.102) (end 181.38 50.38) (width 0.2) (layer "F.Cu") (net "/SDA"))
 (segment (start 194.938 59.58) (end 197.38 59.58) (width 0.2) (layer "F.Cu") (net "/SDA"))
 (segment (start 178.404346 46.5) (end 170 46.5) (width 0.2) (layer "F.Cu") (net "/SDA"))
 (segment (start 167.5 49) (end 167.5 67) (width 0.2) (layer "F.Cu") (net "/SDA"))
 (segment (start 185.31 49.952) (end 184.16 51.102) (width 0.2) (layer "F.Cu") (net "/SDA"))
 (segment (start 167.5 67) (end 162.5 72) (width 0.2) (layer "F.Cu") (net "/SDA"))
 (segment (start 181.38 50.38) (end 181.38 49.475654) (width 0.2) (layer "F.Cu") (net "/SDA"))
 (segment (start 176.76133 48.58067) (end 178.85867 48.58067) (width 0.2) (layer "F.Cu") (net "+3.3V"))
 (segment (start 206.5 58) (end 206.58 58) (width 0.2) (layer "F.Cu") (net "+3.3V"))
 (segment (start 200.934925 72.05) (end 206.5 66.484925) (width 0.2) (layer "F.Cu") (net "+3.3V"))
 (segment (start 200.065075 72.05) (end 200.934925 72.05) (width 0.2) (layer "F.Cu") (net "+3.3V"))
 (segment (start 176 49.342) (end 176.76133 48.58067) (width 0.2) (layer "F.Cu") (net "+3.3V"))
 (segment (start 199.45 71.434925) (end 200.065075 72.05) (width 0.2) (layer "F.Cu") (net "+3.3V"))
 (segment (start 168.784315 45.5) (end 162.5 51.784315) (width 0.2) (layer "F.Cu") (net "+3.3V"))
 (segment (start 162.976346 73.15) (end 176 60.126346) (width 0.2) (layer "F.Cu") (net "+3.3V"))
 (segment (start 178.85867 48.58067) (end 180.23 49.952) (width 0.2) (layer "F.Cu") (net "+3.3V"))
 (segment (start 200.5 68.46) (end 198.738 68.46) (width 0.2) (layer "F.Cu") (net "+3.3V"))
 (segment (start 206.5 66.484925) (end 206.5 58) (width 0.2) (layer "F.Cu") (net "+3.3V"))
 (segment (start 161.35 68.983654) (end 161.35 72.716346) (width 0.2) (layer "F.Cu") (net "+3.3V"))
 (segment (start 200.5 68.46) (end 199.45 69.51) (width 0.2) (layer "F.Cu") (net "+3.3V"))
 (segment (start 162.736346 68.31) (end 162.023654 68.31) (width 0.2) (layer "F.Cu") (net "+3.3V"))
 (segment (start 206.58 58) (end 212.62 51.96) (width 0.2) (layer "F.Cu") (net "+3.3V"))
 (segment (start 161.35 72.716346) (end 161.783654 73.15) (width 0.2) (layer "F.Cu") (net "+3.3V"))
 (segment (start 198.738 68.46) (end 180.23 49.952) (width 0.2) (layer "F.Cu") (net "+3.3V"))
 (segment (start 162.5 64.38) (end 164 65.88) (width 0.2) (layer "F.Cu") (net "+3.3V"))
 (segment (start 164 65.88) (end 164 67.046346) (width 0.2) (layer "F.Cu") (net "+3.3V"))
 (segment (start 176 60.126346) (end 176 49.342) (width 0.2) (layer "F.Cu") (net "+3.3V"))
 (segment (start 184.88 45.5) (end 168.784315 45.5) (width 0.2) (layer "F.Cu") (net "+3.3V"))
 (segment (start 162.5 51.784315) (end 162.5 64.38) (width 0.2) (layer "F.Cu") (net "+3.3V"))
 (segment (start 199.45 69.51) (end 199.45 71.434925) (width 0.2) (layer "F.Cu") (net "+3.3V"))
 (segment (start 164 67.046346) (end 162.736346 68.31) (width 0.2) (layer "F.Cu") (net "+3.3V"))
 (segment (start 162.023654 68.31) (end 161.35 68.983654) (width 0.2) (layer "F.Cu") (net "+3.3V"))
 (segment (start 161.783654 73.15) (end 162.976346 73.15) (width 0.2) (layer "F.Cu") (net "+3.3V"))
 (segment (start 194.25 44.25) (end 191.25 44.25) (width 0.2) (layer "F.Cu") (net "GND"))
 (segment (start 191.25 44.25) (end 180.62 33.62) (width 0.2) (layer "F.Cu") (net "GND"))
 (segment (start 162.5 66.92) (end 160.5 68.92) (width 0.2) (layer "F.Cu") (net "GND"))
 (segment (start 200.5 76.08) (end 211.558 65.022) (width 0.2) (layer "F.Cu") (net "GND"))
 (segment (start 176.03 33.62) (end 171.69 37.96) (width 0.2) (layer "F.Cu") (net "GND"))
 (segment (start 213.455 49.42) (end 212.62 49.42) (width 0.2) (layer "F.Cu") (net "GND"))
 (segment (start 162.5 66.5) (end 162.5 66.92) (width 0.2) (layer "F.Cu") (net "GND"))
 (segment (start 213.69763 49.42) (end 214.971 50.69337) (width 0.2) (layer "F.Cu") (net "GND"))
 (segment (start 156.19 50.46) (end 156.19 60.61) (width 0.2) (layer "F.Cu") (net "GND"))
 (segment (start 214.971 50.936) (end 213.455 49.42) (width 0.2) (layer "F.Cu") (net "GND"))
 (segment (start 158 50.5) (end 156.23 50.5) (width 0.2) (layer "F.Cu") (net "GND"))
 (segment (start 156.23 50.5) (end 156.19 50.46) (width 0.2) (layer "F.Cu") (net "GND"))
 (segment (start 209.535 45.5) (end 195.5 45.5) (width 0.2) (layer "F.Cu") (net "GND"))
 (segment (start 214.971 50.69337) (end 214.971 50.936) (width 0.2) (layer "F.Cu") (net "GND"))
 (segment (start 211.5 56.658105) (end 212.596105 55.562) (width 0.2) (layer "F.Cu") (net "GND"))
 (segment (start 164 84.5) (end 165.75 82.75) (width 0.2) (layer "F.Cu") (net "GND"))
 (segment (start 162.5 67) (end 162.5 66.92) (width 0.2) (layer "F.Cu") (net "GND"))
 (segment (start 200.5 76) (end 200.5 76.08) (width 0.2) (layer "F.Cu") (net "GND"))
 (segment (start 211.558 65.022) (end 211.558 57.058) (width 0.2) (layer "F.Cu") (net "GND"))
 (segment (start 180.62 33.62) (end 176.03 33.62) (width 0.2) (layer "F.Cu") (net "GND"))
 (segment (start 160.5 83.5) (end 161.5 84.5) (width 0.2) (layer "F.Cu") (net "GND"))
 (segment (start 158 50.480101) (end 158 50.5) (width 0.2) (layer "F.Cu") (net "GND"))
 (segment (start 165.75 72.75) (end 177.69 60.81) (width 0.2) (layer "F.Cu") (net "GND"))
 (segment (start 214.909 55.562) (end 214.971 55.5) (width 0.2) (layer "F.Cu") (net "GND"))
 (segment (start 214.971 50.936) (end 214.971 55.5) (width 0.2) (layer "F.Cu") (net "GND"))
 (segment (start 168.5 40.722944) (end 167.757157 40.722944) (width 0.2) (layer "F.Cu") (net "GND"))
 (segment (start 211.5 57) (end 211.5 56.658105) (width 0.2) (layer "F.Cu") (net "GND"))
 (segment (start 161.5 84.5) (end 164 84.5) (width 0.2) (layer "F.Cu") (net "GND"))
 (segment (start 212.596105 55.562) (end 214.909 55.562) (width 0.2) (layer "F.Cu") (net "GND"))
 (segment (start 160.5 68.92) (end 160.5 83.5) (width 0.2) (layer "F.Cu") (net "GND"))
 (segment (start 165.75 82.75) (end 165.75 72.75) (width 0.2) (layer "F.Cu") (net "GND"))
 (segment (start 156.19 60.61) (end 162.5 66.92) (width 0.2) (layer "F.Cu") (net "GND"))
 (segment (start 211.558 57.058) (end 211.5 57) (width 0.2) (layer "F.Cu") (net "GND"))
 (segment (start 171.262944 37.96) (end 168.5 40.722944) (width 0.2) (layer "F.Cu") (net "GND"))
 (segment (start 195.5 45.5) (end 194.25 44.25) (width 0.2) (layer "F.Cu") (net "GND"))
 (segment (start 171.69 37.96) (end 171.262944 37.96) (width 0.2) (layer "F.Cu") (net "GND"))
 (segment (start 177.69 60.81) (end 177.69 49.952) (width 0.2) (layer "F.Cu") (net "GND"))
 (segment (start 213.455 49.42) (end 209.535 45.5) (width 0.2) (layer "F.Cu") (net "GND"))
 (segment (start 167.757157 40.722944) (end 158 50.480101) (width 0.2) (layer "F.Cu") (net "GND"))
 (segment (start 212.62 49.42) (end 213.69763 49.42) (width 0.2) (layer "F.Cu") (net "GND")))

